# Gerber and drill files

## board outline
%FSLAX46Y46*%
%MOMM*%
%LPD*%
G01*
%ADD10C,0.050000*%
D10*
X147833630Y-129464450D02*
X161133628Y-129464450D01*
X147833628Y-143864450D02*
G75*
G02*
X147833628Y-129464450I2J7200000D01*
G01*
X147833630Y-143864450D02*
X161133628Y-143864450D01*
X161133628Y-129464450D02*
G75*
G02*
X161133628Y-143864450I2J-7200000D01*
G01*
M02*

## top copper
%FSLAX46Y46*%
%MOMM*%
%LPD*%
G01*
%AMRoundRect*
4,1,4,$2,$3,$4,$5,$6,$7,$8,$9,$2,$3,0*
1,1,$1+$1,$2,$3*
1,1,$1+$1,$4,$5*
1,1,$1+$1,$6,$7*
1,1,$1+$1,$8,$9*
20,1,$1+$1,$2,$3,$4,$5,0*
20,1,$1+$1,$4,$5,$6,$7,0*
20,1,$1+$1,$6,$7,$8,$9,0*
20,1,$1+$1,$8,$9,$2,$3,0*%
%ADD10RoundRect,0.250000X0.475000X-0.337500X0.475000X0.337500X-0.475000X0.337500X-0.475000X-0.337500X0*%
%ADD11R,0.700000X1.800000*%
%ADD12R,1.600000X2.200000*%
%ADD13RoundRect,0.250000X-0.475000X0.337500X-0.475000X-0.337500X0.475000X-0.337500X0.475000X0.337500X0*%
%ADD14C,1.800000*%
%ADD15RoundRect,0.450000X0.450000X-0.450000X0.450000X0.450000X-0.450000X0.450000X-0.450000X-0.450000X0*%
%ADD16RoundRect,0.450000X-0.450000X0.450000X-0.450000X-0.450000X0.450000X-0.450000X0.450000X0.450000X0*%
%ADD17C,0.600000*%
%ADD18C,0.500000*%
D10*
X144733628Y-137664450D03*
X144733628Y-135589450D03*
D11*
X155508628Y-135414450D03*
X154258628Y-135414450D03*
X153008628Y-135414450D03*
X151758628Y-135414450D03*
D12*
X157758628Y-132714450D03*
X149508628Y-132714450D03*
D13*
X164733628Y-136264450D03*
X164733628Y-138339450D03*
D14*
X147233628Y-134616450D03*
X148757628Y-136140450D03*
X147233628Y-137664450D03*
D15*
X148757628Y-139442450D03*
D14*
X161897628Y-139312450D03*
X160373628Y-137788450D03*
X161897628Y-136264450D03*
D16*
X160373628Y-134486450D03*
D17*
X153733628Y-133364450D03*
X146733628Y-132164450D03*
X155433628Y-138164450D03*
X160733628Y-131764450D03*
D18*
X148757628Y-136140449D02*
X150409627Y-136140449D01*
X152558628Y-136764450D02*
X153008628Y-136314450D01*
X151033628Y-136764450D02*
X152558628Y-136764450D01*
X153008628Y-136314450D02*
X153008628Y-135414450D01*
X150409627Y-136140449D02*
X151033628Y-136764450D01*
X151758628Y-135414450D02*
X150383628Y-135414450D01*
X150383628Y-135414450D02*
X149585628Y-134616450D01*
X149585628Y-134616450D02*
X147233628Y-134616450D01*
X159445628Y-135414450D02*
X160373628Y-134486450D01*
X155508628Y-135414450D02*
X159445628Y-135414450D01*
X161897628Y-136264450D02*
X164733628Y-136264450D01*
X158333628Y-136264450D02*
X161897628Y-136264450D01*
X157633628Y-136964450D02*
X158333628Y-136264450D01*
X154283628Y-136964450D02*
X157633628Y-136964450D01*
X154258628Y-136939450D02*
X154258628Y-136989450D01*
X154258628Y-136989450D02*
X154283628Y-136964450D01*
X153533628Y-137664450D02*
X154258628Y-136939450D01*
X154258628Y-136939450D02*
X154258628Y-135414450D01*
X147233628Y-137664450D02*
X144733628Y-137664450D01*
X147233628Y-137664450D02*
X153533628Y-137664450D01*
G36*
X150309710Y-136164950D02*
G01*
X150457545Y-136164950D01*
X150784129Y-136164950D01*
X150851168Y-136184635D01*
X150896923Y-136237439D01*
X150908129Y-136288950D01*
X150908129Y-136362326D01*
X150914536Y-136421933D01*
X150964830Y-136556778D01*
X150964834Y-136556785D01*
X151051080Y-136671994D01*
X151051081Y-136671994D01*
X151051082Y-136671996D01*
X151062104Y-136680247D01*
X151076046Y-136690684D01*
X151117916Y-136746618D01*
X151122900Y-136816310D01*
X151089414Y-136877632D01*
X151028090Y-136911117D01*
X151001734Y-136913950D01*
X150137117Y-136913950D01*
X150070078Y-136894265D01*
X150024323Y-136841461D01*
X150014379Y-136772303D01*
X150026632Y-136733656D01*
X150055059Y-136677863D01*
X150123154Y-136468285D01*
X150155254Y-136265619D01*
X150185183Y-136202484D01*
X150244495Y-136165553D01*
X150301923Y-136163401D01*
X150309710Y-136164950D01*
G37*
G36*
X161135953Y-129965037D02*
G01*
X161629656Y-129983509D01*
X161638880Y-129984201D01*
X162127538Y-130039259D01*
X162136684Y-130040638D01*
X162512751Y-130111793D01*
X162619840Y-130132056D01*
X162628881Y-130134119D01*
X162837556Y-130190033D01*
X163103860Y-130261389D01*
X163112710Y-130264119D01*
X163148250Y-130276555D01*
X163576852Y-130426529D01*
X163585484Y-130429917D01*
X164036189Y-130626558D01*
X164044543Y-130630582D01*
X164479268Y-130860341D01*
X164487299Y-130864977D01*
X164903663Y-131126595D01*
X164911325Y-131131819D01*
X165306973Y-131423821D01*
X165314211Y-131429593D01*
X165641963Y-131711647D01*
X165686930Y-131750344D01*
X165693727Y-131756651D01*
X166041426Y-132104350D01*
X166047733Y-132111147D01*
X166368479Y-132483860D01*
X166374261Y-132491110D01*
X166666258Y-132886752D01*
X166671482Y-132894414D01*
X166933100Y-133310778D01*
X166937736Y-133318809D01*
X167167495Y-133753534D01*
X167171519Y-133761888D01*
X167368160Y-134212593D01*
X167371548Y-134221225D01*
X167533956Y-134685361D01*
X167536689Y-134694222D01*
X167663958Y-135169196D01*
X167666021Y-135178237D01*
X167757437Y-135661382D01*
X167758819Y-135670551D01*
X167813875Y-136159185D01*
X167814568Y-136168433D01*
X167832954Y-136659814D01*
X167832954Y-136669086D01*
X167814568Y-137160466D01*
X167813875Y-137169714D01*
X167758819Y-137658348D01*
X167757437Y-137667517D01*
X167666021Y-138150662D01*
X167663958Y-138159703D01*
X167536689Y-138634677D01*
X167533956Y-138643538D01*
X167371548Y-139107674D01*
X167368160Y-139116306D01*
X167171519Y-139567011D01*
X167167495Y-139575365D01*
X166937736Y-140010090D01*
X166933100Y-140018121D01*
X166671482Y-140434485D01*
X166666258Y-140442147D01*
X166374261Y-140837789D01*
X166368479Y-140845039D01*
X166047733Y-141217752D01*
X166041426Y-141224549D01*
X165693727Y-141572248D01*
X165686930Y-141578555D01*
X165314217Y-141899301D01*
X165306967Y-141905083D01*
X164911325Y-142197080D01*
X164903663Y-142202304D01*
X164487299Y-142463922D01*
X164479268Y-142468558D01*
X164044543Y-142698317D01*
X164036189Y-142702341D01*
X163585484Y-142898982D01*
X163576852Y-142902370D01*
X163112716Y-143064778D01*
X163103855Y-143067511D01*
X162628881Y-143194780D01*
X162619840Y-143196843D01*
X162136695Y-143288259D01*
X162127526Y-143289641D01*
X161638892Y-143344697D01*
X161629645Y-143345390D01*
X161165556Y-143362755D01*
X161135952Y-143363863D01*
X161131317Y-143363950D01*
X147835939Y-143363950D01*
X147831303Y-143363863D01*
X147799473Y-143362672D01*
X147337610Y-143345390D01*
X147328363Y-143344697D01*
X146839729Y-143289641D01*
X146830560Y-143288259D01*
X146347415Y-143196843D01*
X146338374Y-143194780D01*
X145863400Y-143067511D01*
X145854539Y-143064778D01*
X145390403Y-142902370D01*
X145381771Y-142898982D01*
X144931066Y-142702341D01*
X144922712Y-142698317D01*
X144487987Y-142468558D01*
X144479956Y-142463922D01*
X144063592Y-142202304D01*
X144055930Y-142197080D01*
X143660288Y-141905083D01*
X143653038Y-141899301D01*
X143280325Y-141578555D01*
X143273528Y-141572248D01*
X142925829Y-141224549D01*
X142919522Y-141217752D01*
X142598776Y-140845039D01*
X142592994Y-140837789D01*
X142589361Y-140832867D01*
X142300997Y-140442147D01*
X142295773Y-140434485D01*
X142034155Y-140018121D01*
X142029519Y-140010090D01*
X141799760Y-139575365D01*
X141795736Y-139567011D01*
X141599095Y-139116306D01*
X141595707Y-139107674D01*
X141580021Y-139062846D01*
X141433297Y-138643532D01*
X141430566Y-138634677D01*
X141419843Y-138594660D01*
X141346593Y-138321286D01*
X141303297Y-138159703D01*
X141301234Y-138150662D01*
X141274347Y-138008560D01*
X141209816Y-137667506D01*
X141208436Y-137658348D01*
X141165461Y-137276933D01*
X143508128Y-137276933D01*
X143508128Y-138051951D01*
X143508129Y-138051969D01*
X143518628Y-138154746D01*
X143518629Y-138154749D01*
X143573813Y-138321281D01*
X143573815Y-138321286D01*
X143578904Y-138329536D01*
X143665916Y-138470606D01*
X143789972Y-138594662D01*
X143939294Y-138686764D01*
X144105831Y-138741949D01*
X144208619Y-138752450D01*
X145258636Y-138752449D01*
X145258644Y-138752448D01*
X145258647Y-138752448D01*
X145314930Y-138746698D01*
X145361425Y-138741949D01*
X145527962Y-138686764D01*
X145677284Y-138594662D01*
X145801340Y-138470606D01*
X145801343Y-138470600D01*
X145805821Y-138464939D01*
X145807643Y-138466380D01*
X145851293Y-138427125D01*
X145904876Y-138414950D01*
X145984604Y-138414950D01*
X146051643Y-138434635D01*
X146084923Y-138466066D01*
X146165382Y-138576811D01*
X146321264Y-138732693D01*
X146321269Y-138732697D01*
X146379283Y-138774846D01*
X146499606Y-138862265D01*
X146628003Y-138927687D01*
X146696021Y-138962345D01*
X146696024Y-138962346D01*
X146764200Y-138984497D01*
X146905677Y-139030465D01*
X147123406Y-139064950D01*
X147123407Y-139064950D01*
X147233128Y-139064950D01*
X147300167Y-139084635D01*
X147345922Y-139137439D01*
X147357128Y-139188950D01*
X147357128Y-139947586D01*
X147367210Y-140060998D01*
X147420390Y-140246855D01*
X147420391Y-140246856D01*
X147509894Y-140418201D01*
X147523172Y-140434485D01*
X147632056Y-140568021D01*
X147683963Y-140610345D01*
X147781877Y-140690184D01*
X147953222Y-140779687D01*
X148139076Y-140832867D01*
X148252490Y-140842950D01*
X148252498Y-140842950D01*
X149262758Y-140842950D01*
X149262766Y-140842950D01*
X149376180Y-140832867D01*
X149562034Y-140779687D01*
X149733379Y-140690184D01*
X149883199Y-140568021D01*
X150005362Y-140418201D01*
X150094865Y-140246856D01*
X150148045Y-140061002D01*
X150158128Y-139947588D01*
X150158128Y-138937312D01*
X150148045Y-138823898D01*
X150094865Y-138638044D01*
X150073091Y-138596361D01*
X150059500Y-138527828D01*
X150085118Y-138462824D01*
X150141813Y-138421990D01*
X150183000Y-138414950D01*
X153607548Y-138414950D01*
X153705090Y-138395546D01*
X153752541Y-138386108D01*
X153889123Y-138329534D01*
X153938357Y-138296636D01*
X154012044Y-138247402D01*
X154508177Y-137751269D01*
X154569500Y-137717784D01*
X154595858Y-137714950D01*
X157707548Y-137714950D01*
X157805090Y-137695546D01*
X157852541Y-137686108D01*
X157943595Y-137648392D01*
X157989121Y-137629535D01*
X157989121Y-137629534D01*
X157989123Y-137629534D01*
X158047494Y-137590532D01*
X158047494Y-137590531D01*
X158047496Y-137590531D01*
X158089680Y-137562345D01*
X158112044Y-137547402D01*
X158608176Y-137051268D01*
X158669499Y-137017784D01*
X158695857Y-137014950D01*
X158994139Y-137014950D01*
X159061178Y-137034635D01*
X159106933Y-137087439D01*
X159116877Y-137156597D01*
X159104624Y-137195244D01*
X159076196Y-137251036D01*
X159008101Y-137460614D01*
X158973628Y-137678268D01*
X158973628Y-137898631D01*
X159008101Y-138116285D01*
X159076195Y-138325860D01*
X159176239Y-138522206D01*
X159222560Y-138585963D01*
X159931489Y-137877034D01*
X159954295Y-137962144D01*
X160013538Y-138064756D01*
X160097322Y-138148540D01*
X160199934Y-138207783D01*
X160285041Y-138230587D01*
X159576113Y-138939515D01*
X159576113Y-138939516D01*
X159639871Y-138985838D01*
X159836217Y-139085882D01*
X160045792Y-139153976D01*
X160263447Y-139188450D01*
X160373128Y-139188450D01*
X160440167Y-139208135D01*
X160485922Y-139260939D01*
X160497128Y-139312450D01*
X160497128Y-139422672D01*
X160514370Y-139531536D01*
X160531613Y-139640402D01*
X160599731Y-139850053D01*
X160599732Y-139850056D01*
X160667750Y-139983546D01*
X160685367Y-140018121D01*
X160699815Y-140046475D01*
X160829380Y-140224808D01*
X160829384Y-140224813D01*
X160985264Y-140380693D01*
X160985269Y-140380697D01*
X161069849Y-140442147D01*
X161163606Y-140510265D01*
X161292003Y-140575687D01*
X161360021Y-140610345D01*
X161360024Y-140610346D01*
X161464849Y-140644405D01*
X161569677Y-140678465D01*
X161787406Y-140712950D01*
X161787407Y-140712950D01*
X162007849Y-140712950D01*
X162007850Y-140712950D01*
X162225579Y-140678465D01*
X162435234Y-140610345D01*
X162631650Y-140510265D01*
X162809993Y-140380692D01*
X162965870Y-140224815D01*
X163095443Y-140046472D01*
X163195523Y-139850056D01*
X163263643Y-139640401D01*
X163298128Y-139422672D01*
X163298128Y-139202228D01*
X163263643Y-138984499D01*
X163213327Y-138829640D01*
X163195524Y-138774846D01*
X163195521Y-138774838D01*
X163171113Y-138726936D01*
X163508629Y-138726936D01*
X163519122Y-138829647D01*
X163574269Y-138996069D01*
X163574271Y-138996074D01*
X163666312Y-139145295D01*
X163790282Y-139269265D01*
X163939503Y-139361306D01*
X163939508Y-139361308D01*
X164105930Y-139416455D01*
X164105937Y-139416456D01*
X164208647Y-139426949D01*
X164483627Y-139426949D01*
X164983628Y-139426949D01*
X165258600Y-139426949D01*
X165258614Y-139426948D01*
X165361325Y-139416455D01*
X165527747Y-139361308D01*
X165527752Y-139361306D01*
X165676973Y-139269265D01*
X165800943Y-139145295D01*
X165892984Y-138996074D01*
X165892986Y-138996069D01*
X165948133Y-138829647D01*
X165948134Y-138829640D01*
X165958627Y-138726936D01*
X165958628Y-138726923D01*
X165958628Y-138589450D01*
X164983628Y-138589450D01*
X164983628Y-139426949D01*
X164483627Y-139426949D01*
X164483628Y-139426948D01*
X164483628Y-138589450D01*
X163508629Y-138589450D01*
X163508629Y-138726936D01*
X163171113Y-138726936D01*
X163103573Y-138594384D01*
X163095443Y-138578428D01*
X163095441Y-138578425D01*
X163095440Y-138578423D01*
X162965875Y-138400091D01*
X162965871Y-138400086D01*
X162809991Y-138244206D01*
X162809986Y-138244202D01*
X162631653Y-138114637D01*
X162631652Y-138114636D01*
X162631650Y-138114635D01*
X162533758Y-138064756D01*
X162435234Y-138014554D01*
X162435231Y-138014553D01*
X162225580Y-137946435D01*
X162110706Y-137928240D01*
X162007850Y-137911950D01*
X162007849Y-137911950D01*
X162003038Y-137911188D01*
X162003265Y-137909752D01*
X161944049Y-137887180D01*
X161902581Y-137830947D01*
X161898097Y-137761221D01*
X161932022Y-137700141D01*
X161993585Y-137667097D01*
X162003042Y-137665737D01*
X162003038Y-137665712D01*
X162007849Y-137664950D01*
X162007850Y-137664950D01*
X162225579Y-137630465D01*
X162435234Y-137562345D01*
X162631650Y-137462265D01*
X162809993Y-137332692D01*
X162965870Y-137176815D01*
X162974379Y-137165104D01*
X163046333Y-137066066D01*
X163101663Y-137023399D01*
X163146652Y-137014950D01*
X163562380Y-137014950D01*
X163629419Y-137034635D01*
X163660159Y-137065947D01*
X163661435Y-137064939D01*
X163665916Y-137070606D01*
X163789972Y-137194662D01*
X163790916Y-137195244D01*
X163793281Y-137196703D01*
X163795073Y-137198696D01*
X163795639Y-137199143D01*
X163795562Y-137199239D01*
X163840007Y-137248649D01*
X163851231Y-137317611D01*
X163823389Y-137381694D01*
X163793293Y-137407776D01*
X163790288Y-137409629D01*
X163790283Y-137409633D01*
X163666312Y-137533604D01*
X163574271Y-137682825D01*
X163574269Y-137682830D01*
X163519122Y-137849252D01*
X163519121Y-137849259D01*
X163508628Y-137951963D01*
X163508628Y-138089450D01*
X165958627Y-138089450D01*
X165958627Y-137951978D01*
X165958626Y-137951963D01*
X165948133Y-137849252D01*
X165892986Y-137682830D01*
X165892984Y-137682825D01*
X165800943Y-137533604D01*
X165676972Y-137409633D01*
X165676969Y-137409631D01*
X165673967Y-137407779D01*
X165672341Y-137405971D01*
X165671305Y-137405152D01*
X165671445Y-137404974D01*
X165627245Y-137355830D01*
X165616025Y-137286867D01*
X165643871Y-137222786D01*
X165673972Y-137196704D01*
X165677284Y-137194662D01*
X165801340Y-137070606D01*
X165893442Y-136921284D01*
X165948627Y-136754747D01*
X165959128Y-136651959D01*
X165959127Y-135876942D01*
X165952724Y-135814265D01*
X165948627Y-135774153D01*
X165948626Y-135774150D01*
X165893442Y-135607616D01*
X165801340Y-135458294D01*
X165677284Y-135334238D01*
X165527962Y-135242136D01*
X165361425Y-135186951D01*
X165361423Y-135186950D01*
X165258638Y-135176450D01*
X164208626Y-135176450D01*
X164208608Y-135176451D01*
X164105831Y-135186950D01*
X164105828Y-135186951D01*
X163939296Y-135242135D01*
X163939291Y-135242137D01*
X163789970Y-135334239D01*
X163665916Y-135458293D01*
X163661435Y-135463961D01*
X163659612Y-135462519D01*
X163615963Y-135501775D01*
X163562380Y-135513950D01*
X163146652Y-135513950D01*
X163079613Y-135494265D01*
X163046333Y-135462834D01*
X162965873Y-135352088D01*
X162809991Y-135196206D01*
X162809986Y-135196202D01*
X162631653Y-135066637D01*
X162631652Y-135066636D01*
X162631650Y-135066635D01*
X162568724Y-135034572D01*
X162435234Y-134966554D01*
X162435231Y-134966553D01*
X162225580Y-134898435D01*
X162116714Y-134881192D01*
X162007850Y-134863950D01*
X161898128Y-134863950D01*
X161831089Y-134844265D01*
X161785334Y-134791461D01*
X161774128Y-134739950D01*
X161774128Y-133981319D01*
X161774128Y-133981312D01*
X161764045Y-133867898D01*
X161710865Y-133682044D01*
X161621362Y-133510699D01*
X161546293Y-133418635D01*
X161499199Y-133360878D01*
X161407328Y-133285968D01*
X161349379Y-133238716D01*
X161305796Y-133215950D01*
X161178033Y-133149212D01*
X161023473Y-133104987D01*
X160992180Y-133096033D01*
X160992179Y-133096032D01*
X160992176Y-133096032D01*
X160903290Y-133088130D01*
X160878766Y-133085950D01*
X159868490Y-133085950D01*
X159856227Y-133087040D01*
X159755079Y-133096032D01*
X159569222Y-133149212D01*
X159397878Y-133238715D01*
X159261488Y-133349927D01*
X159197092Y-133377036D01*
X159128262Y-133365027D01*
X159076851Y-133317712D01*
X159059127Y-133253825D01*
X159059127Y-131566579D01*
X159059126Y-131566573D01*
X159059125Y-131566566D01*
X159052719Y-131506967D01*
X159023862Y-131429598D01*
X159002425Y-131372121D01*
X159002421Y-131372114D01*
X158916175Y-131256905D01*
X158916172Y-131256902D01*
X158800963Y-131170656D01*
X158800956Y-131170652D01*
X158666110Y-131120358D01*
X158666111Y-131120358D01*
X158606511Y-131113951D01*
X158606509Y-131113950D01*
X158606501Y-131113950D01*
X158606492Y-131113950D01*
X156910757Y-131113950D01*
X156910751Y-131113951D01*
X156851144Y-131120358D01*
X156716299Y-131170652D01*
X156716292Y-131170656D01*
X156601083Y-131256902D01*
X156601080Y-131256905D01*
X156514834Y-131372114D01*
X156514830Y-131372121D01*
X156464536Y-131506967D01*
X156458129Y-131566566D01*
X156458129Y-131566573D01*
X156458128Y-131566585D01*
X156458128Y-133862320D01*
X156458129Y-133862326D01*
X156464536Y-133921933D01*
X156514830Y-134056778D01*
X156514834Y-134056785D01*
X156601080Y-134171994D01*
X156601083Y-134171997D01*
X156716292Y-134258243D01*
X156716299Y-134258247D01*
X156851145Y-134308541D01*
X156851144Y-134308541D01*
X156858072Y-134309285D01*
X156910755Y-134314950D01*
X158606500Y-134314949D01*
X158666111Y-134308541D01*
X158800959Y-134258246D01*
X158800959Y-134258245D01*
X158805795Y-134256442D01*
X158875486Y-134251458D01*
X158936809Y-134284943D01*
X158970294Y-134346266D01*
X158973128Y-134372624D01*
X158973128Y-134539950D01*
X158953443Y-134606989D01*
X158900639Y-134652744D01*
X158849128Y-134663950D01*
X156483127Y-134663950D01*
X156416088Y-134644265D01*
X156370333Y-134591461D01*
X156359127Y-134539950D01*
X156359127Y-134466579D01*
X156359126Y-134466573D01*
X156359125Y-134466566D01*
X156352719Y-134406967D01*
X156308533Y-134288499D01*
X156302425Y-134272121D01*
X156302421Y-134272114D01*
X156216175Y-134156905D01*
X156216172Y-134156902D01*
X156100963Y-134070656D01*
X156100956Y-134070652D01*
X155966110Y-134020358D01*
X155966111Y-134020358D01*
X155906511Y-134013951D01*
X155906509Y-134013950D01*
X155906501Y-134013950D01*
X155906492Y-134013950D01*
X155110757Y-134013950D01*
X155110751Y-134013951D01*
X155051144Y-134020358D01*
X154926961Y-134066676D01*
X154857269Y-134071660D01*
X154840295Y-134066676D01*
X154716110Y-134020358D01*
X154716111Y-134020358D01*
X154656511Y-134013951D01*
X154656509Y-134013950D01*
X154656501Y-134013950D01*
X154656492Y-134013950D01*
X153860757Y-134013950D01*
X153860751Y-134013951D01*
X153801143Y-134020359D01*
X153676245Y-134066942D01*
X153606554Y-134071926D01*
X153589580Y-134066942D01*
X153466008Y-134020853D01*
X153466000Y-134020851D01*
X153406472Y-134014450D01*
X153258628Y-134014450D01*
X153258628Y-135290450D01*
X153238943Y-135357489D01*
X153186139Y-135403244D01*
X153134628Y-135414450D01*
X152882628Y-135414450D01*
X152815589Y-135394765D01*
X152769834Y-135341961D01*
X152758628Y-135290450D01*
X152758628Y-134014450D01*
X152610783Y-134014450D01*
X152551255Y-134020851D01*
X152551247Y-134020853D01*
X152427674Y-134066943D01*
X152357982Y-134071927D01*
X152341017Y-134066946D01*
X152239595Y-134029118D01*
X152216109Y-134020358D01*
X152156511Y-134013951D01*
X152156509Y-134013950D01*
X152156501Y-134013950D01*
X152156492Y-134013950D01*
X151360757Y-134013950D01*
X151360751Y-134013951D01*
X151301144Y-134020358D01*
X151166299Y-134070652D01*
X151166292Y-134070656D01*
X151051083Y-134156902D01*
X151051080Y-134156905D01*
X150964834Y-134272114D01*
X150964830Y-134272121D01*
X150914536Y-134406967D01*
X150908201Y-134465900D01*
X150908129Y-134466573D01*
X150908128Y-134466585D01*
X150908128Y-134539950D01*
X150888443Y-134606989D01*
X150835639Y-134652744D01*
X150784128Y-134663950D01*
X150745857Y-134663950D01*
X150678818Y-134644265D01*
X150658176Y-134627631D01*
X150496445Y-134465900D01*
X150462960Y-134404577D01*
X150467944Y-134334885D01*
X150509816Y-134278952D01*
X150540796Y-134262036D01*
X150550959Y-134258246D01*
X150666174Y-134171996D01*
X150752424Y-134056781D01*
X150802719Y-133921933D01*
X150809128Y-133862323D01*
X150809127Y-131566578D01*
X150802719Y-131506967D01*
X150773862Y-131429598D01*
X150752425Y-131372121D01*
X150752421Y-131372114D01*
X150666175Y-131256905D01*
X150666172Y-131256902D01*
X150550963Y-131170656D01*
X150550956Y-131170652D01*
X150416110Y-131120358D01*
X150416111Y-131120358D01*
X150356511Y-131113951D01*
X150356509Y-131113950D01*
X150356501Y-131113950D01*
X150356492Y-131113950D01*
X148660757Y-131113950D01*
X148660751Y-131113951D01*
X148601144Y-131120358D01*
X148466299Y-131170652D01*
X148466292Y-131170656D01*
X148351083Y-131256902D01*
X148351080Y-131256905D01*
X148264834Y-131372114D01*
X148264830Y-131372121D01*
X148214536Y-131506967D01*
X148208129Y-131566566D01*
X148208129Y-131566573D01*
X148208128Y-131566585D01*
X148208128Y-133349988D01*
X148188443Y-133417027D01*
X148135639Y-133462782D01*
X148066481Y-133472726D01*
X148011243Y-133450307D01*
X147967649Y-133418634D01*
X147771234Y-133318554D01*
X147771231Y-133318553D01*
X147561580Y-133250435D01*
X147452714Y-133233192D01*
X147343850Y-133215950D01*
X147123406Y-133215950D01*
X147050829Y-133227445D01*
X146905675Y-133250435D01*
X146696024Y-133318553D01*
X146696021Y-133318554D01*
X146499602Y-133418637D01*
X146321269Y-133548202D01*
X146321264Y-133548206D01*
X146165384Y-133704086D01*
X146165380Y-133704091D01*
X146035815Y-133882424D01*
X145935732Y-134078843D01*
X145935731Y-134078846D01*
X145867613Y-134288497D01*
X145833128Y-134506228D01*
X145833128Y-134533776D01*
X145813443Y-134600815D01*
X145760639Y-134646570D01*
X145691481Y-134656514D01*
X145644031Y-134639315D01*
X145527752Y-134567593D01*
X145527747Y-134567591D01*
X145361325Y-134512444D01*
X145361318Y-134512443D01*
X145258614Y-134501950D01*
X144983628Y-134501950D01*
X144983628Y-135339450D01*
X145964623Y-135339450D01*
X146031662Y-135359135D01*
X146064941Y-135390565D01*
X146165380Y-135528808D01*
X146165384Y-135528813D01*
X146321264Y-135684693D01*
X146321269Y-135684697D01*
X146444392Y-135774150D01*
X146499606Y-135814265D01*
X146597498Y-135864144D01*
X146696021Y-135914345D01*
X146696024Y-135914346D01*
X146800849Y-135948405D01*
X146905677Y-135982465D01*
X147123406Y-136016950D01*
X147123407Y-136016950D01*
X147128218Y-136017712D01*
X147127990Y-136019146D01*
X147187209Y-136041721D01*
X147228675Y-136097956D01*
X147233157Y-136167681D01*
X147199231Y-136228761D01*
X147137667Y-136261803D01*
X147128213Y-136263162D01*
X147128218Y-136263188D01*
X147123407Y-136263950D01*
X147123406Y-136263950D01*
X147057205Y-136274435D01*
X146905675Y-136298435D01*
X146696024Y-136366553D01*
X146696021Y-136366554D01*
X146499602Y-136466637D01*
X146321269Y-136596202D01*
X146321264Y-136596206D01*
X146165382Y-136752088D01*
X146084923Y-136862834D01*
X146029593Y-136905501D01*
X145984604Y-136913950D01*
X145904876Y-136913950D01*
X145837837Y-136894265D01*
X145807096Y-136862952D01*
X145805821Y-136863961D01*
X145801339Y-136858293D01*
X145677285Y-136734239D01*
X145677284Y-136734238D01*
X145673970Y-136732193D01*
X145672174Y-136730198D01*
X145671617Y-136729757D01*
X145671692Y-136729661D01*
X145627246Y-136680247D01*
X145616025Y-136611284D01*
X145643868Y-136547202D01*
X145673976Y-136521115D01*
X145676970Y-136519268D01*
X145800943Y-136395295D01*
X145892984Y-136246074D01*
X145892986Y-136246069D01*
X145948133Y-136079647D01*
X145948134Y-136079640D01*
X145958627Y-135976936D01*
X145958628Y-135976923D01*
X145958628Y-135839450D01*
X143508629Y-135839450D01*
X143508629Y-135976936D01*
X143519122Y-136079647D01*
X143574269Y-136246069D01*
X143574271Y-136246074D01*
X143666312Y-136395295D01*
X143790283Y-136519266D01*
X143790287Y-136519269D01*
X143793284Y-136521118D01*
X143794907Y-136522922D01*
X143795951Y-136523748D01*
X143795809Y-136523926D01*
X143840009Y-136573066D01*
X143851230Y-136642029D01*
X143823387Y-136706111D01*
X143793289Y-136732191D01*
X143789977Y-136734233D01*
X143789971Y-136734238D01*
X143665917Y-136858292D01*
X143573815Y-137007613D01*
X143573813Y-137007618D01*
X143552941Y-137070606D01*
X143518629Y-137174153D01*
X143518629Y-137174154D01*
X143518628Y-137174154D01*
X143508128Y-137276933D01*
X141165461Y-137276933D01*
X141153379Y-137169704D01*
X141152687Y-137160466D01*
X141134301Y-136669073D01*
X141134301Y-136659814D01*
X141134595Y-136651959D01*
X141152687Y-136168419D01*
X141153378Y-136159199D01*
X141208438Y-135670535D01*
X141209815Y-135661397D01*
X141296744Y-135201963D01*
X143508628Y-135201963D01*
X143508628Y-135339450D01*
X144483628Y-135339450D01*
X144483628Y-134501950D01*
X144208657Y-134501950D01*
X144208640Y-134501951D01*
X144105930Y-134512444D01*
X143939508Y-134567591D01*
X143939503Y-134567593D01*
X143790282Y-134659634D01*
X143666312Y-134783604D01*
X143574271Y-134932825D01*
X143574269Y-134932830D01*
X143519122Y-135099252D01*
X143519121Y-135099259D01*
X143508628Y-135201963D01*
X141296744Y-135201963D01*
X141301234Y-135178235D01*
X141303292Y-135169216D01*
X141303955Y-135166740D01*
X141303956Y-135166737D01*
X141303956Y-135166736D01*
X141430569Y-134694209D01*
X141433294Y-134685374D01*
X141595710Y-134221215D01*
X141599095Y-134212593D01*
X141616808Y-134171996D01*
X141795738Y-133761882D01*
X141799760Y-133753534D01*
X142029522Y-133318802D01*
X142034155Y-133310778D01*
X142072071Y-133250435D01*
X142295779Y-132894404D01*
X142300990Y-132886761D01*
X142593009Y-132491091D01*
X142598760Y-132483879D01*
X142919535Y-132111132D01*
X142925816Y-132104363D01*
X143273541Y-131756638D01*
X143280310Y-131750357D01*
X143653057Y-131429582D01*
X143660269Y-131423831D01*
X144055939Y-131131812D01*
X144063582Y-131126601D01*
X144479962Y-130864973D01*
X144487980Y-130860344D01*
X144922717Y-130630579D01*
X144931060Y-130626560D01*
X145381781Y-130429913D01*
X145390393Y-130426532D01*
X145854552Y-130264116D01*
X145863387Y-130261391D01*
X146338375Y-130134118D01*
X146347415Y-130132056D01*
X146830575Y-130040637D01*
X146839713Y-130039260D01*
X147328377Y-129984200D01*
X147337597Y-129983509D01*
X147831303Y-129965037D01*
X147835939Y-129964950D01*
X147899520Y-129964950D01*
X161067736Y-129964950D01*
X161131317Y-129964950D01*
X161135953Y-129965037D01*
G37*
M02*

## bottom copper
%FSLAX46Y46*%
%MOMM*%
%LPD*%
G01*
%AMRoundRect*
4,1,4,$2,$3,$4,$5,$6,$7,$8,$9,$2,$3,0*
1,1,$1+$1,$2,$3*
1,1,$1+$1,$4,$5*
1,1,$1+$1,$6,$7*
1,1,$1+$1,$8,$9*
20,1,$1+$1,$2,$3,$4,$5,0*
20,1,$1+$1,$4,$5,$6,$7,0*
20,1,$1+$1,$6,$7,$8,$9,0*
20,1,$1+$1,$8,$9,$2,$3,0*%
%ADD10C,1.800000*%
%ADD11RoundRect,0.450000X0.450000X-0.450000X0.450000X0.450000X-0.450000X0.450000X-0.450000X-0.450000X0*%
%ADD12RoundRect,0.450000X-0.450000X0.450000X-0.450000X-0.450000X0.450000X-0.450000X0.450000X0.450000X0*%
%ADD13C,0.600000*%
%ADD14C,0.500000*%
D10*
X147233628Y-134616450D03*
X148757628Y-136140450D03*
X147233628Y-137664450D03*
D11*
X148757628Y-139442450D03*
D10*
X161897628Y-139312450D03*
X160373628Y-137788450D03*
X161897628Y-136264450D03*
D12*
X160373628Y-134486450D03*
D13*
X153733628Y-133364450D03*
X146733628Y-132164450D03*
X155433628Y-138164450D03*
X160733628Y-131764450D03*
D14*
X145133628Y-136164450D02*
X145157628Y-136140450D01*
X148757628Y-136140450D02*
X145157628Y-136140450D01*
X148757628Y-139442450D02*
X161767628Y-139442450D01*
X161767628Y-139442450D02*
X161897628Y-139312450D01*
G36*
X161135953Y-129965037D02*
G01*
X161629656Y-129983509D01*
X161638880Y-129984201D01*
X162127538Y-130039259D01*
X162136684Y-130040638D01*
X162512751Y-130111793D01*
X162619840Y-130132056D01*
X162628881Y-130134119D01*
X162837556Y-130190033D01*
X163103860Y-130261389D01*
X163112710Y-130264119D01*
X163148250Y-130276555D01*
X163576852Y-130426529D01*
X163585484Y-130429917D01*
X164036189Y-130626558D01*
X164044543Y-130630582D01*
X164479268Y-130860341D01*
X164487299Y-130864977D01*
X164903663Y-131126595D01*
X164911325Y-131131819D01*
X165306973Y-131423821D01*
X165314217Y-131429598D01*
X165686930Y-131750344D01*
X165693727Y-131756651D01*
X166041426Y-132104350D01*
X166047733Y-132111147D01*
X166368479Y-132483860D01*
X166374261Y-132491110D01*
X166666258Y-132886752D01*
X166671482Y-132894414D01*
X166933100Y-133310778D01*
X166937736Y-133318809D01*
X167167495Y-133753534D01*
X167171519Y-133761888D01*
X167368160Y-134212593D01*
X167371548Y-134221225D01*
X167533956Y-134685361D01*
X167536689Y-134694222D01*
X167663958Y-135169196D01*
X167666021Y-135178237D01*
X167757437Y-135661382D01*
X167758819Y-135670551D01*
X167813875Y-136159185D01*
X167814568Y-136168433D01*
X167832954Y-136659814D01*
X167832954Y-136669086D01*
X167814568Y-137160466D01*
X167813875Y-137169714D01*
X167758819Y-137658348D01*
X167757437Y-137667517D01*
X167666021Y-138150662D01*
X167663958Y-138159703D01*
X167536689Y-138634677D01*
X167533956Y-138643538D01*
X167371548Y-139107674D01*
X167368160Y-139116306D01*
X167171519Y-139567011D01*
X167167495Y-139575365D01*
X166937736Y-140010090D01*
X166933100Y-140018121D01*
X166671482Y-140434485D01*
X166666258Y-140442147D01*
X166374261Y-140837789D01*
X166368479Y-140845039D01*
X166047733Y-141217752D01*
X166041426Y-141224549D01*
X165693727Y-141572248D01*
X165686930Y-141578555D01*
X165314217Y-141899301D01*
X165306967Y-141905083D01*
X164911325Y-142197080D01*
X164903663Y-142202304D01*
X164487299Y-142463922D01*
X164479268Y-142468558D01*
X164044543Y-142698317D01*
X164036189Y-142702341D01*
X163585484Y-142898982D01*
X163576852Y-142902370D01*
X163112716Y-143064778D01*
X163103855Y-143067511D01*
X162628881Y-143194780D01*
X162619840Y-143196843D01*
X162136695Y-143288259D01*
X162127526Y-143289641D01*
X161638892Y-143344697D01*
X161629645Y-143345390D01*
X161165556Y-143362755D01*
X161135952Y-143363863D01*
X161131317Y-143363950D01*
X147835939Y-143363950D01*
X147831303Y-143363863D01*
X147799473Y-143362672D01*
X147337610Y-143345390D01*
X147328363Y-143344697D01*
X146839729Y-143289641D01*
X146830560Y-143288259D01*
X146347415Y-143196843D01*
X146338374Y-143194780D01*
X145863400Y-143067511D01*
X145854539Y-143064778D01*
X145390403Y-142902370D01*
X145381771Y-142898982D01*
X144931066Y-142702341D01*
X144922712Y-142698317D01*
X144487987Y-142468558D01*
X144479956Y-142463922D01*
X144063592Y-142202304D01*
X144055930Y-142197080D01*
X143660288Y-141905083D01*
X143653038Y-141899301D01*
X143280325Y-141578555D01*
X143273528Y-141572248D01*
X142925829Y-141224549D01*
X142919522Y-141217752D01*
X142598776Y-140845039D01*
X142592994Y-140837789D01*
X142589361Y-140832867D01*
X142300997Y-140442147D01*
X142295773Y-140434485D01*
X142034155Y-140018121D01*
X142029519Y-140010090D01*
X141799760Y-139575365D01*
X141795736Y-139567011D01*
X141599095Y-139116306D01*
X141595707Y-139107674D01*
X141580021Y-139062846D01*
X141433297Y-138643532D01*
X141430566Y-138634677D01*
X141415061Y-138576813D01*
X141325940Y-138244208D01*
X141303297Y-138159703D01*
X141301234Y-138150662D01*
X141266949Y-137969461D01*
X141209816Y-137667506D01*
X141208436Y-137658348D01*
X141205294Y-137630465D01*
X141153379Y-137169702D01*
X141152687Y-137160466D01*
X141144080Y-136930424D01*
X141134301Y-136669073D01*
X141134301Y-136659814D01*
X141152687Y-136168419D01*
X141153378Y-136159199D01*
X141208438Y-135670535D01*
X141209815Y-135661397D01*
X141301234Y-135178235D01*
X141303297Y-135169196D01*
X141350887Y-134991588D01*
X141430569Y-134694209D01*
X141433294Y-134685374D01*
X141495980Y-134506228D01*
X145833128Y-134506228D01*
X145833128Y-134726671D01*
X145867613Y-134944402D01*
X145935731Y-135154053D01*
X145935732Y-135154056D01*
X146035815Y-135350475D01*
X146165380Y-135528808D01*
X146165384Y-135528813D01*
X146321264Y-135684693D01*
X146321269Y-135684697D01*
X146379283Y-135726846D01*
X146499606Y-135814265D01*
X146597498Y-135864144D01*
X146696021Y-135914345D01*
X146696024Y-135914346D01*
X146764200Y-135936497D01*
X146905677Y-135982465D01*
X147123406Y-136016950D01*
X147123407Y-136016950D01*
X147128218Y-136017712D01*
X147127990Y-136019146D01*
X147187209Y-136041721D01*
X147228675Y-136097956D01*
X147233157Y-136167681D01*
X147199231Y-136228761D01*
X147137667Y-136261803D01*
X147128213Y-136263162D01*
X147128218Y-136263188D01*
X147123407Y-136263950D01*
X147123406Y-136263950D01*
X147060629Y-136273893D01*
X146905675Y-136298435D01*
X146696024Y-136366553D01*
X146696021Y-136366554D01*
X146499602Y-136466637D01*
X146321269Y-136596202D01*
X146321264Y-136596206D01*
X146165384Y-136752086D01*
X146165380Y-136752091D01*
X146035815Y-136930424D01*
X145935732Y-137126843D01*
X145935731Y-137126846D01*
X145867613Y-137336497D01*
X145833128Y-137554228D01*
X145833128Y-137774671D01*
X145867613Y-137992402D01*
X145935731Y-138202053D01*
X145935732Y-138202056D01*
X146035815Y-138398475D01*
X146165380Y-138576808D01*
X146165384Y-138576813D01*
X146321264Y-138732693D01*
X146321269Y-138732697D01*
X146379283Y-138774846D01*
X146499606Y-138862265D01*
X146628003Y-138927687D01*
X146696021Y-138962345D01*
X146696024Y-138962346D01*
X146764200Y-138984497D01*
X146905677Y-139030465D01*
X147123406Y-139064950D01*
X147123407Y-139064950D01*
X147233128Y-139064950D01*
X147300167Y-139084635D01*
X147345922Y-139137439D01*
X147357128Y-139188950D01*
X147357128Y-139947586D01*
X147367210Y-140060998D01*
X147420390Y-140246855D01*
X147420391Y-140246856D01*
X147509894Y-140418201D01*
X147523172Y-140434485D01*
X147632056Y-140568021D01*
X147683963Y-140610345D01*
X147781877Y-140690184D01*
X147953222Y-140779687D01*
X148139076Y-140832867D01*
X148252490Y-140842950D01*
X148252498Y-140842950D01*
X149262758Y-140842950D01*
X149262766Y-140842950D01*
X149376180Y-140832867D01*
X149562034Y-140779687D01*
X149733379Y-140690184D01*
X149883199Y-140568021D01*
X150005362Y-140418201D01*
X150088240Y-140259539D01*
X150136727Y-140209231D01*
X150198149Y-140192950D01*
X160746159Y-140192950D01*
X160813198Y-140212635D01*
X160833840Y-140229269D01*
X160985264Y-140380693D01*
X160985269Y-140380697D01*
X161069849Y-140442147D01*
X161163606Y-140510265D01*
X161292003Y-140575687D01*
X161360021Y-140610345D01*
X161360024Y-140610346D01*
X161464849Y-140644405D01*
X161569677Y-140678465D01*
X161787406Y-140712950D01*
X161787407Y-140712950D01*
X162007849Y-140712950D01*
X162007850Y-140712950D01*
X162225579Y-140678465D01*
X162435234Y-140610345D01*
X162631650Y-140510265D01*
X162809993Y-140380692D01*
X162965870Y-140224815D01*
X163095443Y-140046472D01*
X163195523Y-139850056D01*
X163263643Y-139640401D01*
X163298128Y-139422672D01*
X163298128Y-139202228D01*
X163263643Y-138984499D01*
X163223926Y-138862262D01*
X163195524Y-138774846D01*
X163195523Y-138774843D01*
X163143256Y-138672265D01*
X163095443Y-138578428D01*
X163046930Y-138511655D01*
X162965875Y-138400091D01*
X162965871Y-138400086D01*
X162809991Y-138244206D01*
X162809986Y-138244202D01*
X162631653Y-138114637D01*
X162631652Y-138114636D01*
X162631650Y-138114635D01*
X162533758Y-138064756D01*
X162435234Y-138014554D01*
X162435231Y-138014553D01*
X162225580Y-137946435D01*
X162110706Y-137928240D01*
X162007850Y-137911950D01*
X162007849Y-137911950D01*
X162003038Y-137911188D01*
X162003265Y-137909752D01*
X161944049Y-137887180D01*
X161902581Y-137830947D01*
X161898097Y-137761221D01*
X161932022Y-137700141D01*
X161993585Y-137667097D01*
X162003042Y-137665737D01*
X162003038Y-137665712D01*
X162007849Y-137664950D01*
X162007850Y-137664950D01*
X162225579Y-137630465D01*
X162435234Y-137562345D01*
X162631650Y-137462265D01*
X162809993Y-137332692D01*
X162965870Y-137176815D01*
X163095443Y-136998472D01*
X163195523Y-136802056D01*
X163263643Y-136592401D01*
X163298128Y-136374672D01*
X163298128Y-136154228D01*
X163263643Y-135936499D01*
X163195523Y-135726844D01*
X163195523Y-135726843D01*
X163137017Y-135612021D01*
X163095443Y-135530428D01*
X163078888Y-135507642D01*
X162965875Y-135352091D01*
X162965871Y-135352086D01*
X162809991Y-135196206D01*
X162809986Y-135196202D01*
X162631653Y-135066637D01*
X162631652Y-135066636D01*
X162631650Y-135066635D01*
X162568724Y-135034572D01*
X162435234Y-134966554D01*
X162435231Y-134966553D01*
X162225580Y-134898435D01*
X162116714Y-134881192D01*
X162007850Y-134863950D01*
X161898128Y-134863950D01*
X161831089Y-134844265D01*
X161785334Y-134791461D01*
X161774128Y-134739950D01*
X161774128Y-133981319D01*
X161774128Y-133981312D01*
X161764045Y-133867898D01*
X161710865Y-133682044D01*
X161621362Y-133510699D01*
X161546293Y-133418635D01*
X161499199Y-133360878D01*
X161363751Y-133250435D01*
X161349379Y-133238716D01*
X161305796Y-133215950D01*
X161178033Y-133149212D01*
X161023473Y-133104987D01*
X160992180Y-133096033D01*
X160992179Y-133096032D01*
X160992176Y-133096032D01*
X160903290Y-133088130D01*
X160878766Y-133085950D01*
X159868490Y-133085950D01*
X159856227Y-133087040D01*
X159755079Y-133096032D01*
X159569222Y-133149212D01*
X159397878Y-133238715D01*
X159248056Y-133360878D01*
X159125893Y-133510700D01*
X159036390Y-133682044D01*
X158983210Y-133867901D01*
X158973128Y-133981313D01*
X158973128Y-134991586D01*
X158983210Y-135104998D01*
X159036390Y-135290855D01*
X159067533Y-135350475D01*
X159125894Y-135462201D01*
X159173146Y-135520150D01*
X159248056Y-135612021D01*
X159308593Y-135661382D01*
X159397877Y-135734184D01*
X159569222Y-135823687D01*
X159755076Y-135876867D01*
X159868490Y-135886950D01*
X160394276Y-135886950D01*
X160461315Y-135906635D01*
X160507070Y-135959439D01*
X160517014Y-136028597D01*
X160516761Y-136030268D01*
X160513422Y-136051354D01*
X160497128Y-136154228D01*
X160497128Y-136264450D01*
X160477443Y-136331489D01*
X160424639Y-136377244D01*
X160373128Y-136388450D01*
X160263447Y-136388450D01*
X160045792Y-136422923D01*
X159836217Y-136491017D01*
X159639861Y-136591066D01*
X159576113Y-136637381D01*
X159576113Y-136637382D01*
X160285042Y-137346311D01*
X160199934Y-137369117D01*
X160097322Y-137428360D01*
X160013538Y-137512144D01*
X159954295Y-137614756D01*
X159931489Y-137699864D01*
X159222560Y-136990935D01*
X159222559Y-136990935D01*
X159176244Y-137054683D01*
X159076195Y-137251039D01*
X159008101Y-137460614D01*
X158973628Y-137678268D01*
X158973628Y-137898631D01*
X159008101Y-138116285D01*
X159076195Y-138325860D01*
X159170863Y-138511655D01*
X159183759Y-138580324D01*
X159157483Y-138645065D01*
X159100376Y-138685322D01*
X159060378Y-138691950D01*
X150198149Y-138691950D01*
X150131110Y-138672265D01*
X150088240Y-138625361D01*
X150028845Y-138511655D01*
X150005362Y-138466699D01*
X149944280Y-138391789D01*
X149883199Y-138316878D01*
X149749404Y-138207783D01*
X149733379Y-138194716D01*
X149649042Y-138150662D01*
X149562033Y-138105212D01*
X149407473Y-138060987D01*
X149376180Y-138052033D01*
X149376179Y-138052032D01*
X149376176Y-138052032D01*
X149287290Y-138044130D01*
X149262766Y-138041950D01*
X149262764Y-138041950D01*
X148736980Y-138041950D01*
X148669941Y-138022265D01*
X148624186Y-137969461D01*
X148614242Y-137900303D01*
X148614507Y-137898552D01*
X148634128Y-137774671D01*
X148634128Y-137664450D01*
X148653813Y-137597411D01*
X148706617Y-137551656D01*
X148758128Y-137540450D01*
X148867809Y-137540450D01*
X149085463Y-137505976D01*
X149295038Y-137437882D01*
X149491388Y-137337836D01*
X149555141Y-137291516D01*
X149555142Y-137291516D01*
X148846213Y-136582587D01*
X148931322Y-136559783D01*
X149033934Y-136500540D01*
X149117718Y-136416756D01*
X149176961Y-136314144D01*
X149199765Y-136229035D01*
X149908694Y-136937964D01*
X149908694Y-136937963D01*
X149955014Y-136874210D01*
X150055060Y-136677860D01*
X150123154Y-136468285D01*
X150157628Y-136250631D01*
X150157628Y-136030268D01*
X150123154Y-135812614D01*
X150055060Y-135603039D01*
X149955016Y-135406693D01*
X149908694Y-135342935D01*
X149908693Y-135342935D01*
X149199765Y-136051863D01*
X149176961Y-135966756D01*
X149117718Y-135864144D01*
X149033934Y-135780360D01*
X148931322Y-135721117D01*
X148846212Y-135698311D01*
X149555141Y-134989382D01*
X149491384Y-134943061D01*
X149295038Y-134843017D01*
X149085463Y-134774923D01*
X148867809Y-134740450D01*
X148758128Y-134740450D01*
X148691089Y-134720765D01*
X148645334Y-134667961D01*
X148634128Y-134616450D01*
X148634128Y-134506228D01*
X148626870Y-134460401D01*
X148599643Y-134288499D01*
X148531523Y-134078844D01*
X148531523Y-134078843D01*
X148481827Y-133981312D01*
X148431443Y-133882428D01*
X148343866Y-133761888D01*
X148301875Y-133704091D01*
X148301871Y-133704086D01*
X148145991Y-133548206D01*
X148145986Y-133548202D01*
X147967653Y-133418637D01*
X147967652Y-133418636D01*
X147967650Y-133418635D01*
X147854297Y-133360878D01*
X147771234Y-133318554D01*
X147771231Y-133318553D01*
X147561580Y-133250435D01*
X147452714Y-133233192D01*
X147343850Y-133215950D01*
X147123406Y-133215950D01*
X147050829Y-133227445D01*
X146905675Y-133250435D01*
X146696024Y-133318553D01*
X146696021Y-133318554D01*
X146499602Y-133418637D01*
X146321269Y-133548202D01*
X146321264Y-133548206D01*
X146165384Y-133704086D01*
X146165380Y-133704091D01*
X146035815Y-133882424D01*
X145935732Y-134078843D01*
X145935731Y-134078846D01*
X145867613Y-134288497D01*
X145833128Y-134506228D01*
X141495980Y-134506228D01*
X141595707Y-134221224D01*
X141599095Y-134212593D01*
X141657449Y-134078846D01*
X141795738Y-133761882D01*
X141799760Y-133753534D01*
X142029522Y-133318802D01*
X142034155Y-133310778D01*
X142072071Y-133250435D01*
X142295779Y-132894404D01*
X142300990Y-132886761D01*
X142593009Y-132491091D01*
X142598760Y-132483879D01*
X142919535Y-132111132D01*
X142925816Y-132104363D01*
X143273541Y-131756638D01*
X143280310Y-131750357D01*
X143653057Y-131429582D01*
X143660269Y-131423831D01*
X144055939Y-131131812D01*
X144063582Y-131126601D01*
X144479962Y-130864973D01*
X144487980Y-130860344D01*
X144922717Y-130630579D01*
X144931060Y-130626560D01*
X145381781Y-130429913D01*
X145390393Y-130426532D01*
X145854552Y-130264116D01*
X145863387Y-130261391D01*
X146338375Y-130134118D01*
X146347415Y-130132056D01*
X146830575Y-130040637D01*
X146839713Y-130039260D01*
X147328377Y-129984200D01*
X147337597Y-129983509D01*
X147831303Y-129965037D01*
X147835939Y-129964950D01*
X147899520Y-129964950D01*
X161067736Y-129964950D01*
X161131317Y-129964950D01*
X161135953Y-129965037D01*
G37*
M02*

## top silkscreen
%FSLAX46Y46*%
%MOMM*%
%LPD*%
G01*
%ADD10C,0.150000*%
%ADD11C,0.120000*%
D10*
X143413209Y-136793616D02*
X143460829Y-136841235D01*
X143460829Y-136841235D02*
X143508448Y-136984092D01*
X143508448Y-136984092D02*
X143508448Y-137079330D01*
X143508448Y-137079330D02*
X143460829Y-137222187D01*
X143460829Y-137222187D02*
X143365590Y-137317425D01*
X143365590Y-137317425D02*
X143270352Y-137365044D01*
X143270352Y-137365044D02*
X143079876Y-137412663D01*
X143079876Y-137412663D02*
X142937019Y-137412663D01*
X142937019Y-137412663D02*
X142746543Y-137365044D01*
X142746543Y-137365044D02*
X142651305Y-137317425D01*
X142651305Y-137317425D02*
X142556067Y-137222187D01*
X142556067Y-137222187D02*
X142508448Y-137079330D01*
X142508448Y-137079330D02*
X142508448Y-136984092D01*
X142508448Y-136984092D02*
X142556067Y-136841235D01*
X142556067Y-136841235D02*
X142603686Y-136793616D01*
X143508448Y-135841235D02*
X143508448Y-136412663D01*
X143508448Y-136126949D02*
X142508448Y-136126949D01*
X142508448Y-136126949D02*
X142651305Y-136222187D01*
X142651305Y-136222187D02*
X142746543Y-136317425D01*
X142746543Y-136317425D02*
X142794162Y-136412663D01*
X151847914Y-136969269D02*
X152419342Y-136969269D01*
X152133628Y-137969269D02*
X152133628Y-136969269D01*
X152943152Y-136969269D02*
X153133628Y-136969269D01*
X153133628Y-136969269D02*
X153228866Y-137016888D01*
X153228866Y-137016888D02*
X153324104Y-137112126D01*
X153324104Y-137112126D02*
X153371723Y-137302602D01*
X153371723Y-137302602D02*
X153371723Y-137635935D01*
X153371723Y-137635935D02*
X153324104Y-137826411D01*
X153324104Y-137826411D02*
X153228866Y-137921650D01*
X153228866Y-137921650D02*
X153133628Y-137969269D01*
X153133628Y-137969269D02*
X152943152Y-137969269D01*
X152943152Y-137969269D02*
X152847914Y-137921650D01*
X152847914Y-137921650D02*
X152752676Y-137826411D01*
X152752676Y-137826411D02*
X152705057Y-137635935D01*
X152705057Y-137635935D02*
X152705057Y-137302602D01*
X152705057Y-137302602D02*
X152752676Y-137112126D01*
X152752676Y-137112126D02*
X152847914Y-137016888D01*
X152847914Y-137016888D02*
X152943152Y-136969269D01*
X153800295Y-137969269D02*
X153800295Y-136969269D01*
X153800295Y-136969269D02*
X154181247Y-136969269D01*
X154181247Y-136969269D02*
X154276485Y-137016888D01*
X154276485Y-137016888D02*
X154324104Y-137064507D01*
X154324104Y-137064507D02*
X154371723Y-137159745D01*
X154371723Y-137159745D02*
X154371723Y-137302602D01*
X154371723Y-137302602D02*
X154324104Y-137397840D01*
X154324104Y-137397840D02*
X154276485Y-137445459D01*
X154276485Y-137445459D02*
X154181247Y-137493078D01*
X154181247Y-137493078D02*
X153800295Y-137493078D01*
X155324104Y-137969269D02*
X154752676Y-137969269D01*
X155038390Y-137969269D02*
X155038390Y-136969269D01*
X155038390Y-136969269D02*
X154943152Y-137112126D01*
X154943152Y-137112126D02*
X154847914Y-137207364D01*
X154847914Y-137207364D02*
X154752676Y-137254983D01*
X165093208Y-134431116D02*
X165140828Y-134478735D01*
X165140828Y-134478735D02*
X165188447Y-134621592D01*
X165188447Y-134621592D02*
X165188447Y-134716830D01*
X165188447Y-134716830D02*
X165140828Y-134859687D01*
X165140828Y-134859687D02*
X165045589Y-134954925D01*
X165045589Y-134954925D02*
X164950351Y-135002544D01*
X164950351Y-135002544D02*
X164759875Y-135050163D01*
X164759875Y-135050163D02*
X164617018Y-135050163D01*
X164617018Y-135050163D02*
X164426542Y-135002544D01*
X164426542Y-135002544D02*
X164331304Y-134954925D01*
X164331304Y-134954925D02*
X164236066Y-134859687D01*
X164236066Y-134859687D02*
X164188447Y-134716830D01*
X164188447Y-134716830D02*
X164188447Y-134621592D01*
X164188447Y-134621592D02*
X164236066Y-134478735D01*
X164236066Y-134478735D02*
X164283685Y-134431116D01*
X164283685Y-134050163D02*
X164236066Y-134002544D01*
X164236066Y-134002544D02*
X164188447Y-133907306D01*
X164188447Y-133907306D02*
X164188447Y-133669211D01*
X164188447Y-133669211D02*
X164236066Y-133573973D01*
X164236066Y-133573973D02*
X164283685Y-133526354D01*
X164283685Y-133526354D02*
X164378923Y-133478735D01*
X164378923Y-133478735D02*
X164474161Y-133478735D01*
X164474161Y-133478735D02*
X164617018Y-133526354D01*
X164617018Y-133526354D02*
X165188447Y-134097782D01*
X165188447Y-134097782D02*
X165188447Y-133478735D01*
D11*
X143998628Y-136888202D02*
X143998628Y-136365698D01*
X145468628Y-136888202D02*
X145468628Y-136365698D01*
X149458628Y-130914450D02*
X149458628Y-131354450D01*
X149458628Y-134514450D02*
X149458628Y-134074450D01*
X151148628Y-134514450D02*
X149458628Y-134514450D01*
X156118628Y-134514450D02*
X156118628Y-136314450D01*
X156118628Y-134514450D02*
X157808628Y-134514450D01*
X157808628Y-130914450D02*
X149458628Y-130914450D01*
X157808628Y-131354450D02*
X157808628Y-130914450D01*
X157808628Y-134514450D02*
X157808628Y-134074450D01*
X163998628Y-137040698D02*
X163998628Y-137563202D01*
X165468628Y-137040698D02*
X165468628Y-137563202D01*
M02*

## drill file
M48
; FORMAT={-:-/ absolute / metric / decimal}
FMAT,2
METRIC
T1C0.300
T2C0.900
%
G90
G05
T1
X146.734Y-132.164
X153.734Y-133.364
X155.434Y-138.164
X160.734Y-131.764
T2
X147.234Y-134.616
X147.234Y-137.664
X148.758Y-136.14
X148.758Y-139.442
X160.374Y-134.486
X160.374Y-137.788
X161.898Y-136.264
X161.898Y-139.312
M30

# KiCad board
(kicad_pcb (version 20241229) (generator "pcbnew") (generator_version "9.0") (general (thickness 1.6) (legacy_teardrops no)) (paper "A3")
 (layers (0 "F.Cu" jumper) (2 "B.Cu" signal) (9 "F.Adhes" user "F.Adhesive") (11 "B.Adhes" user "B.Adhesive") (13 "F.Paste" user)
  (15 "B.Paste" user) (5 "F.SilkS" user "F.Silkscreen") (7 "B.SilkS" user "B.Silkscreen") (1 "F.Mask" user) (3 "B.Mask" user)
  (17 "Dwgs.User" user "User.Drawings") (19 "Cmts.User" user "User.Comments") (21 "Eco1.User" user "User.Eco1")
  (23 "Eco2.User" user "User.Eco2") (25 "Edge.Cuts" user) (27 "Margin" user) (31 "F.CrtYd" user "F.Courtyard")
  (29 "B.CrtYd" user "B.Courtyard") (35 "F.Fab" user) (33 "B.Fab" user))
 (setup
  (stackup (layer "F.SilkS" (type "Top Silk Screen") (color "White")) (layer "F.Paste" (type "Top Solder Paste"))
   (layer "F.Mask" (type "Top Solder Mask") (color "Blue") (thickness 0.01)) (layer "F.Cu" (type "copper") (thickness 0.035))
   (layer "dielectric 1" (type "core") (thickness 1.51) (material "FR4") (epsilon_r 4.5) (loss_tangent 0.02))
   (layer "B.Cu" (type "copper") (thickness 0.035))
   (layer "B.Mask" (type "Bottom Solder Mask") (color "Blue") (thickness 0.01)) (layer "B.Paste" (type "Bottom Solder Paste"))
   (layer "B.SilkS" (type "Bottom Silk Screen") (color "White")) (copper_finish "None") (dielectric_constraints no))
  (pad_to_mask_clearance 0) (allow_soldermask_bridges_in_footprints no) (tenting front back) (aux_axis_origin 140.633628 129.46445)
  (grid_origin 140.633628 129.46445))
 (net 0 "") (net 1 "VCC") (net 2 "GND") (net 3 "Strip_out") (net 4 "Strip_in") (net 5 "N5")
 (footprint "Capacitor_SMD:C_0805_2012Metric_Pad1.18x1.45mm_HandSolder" (layer "F.Cu") (at 144.733628 136.62695 90)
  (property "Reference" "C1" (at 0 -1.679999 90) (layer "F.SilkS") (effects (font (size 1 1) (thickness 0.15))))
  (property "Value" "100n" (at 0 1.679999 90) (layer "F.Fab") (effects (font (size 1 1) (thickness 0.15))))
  (fp_line (start -0.261252 -0.735) (end 0.261252 -0.735) (stroke (width 0.12) (type solid)) (layer "F.SilkS"))
  (fp_line (start -0.261252 0.735) (end 0.261252 0.735) (stroke (width 0.12) (type solid)) (layer "F.SilkS"))
  (pad "1" smd roundrect (at -1.0375 0 90) (size 1.175 1.45) (layers "F.Cu" "F.Mask" "F.Paste") (roundrect_rratio 0.212766) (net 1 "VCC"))
  (pad "2" smd roundrect (at 1.0375 0 90) (size 1.175 1.45) (layers "F.Cu" "F.Mask" "F.Paste") (roundrect_rratio 0.212766) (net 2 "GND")))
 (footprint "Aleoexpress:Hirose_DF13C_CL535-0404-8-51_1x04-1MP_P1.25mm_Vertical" (layer "F.Cu") (at 153.633628 133.96445 180)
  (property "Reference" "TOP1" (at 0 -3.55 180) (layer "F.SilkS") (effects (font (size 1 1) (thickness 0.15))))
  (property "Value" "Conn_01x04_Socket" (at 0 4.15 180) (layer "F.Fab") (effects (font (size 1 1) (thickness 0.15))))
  (fp_line (start 4.175 3.05) (end 4.175 2.61) (stroke (width 0.12) (type solid)) (layer "F.SilkS"))
  (fp_line (start 4.175 -0.55) (end 4.175 -0.11) (stroke (width 0.12) (type solid)) (layer "F.SilkS"))
  (fp_line (start 2.485 -0.55) (end 4.175 -0.55) (stroke (width 0.12) (type solid)) (layer "F.SilkS"))
  (fp_line (start -2.485 -0.55) (end -2.485 -2.35) (stroke (width 0.12) (type solid)) (layer "F.SilkS"))
  (fp_line (start -2.485 -0.55) (end -4.175 -0.55) (stroke (width 0.12) (type solid)) (layer "F.SilkS"))
  (fp_line (start -4.175 3.05) (end 4.175 3.05) (stroke (width 0.12) (type solid)) (layer "F.SilkS"))
  (fp_line (start -4.175 2.61) (end -4.175 3.05) (stroke (width 0.12) (type solid)) (layer "F.SilkS"))
  (fp_line (start -4.175 -0.55) (end -4.175 -0.11) (stroke (width 0.12) (type solid)) (layer "F.SilkS"))
  (pad "1" smd rect (at -1.875 -1.45 180) (size 0.7 1.8) (layers "F.Cu" "F.Mask" "F.Paste") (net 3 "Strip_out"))
  (pad "2" smd rect (at -0.625 -1.45 180) (size 0.7 1.8) (layers "F.Cu" "F.Mask" "F.Paste") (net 1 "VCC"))
  (pad "3" smd rect (at 0.625 -1.45 180) (size 0.7 1.8) (layers "F.Cu" "F.Mask" "F.Paste") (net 2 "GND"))
  (pad "4" smd rect (at 1.875 -1.45 180) (size 0.7 1.8) (layers "F.Cu" "F.Mask" "F.Paste") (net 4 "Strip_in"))
  (pad "MP" smd rect (at -4.125 1.25 180) (size 1.6 2.2) (layers "F.Cu" "F.Mask" "F.Paste"))
  (pad "MP" smd rect (at 4.125 1.25 180) (size 1.6 2.2) (layers "F.Cu" "F.Mask" "F.Paste")))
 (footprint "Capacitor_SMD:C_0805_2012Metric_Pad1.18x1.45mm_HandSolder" (layer "F.Cu") (at 164.733628 137.30195 -90)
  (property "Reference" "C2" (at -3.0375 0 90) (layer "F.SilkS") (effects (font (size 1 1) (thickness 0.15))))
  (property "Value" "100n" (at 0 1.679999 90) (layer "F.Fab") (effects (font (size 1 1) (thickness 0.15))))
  (fp_line (start -0.261252 0.735) (end 0.261252 0.735) (stroke (width 0.12) (type solid)) (layer "F.SilkS"))
  (fp_line (start -0.261252 -0.735) (end 0.261252 -0.735) (stroke (width 0.12) (type solid)) (layer "F.SilkS"))
  (pad "1" smd roundrect (at -1.0375 0 270) (size 1.175 1.45) (layers "F.Cu" "F.Mask" "F.Paste") (roundrect_rratio 0.212766) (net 1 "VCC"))
  (pad "2" smd roundrect (at 1.0375 0 270) (size 1.175 1.45) (layers "F.Cu" "F.Mask" "F.Paste") (roundrect_rratio 0.212766) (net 2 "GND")))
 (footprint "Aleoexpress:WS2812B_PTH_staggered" (layer "B.Cu") (at 148.757628 139.44245 90)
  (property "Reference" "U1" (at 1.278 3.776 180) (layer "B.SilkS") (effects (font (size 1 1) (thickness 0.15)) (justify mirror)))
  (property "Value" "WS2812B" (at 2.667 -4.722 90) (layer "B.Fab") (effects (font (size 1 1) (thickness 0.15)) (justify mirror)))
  (pad "1" thru_hole circle (at 4.826 -1.524 90) (size 1.8 1.8) (drill 0.9) (layers "*.Cu" "*.Mask") (remove_unused_layers no)
   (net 4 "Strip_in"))
  (pad "2" thru_hole circle (at 3.302 0 90) (size 1.8 1.8) (drill 0.9) (layers "*.Cu" "*.Mask") (remove_unused_layers no) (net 2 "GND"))
  (pad "3" thru_hole circle (at 1.778 -1.524 90) (size 1.8 1.8) (drill 0.9) (layers "*.Cu" "*.Mask") (remove_unused_layers no) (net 1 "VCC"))
  (pad "4" thru_hole roundrect (at 0 0 90) (size 1.8 1.8) (drill 0.9) (layers "*.Cu" "*.Mask") (remove_unused_layers no)
   (roundrect_rratio 0.25) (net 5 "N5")))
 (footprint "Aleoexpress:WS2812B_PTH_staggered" (layer "B.Cu") (at 160.373628 134.48645 -90)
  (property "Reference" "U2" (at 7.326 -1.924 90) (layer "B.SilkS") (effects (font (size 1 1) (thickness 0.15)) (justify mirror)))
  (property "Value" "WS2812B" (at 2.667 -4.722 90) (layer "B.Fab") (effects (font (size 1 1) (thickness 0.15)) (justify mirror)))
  (pad "1" thru_hole circle (at 4.826 -1.524 270) (size 1.8 1.8) (drill 0.9) (layers "*.Cu" "*.Mask") (remove_unused_layers no) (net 5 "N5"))
  (pad "2" thru_hole circle (at 3.302 0 270) (size 1.8 1.8) (drill 0.9) (layers "*.Cu" "*.Mask") (remove_unused_layers no) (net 2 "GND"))
  (pad "3" thru_hole circle (at 1.778 -1.524 270) (size 1.8 1.8) (drill 0.9) (layers "*.Cu" "*.Mask") (remove_unused_layers no)
   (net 1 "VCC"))
  (pad "4" thru_hole roundrect (at 0 0 270) (size 1.8 1.8) (drill 0.9) (layers "*.Cu" "*.Mask") (remove_unused_layers no)
   (roundrect_rratio 0.25) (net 3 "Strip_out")))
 (gr_line (start 147.83363 129.46445) (end 161.133628 129.46445) (stroke (width 0.05) (type default)) (layer "Edge.Cuts"))
 (gr_arc (start 147.833628 143.86445) (mid 140.633628 136.66445) (end 147.833628 129.46445) (stroke (width 0.05) (type default))
  (layer "Edge.Cuts"))
 (gr_line (start 147.83363 143.86445) (end 161.133628 143.86445) (stroke (width 0.05) (type default)) (layer "Edge.Cuts"))
 (gr_arc (start 161.133628 129.46445) (mid 168.333628 136.66445) (end 161.133628 143.86445) (stroke (width 0.05) (type default))
  (layer "Edge.Cuts"))
 (segment (start 148.757628 136.140449) (end 150.409627 136.140449) (width 0.5) (layer "F.Cu") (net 2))
 (segment (start 152.558628 136.76445) (end 153.008628 136.31445) (width 0.5) (layer "F.Cu") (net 2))
 (segment (start 151.033628 136.76445) (end 152.558628 136.76445) (width 0.5) (layer "F.Cu") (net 2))
 (segment (start 153.008628 136.31445) (end 153.008628 135.41445) (width 0.5) (layer "F.Cu") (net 2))
 (segment (start 150.409627 136.140449) (end 151.033628 136.76445) (width 0.5) (layer "F.Cu") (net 2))
 (via (at 153.733628 133.36445) (size 0.6) (drill 0.3) (layers "F.Cu" "B.Cu") (free yes) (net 2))
 (via (at 146.733628 132.16445) (size 0.6) (drill 0.3) (layers "F.Cu" "B.Cu") (free yes) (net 2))
 (via (at 155.433628 138.16445) (size 0.6) (drill 0.3) (layers "F.Cu" "B.Cu") (free yes) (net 2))
 (via (at 160.733628 131.76445) (size 0.6) (drill 0.3) (layers "F.Cu" "B.Cu") (free yes) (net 2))
 (segment (start 145.133628 136.16445) (end 145.157628 136.14045) (width 0.5) (layer "B.Cu") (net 2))
 (segment (start 148.757628 136.14045) (end 145.157628 136.14045) (width 0.5) (layer "B.Cu") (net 2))
 (segment (start 151.758628 135.41445) (end 150.383628 135.41445) (width 0.5) (layer "F.Cu") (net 4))
 (segment (start 150.383628 135.41445) (end 149.585628 134.61645) (width 0.5) (layer "F.Cu") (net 4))
 (segment (start 149.585628 134.61645) (end 147.233628 134.61645) (width 0.5) (layer "F.Cu") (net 4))
 (segment (start 148.757628 139.44245) (end 161.767628 139.44245) (width 0.5) (layer "B.Cu") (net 5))
 (segment (start 161.767628 139.44245) (end 161.897628 139.31245) (width 0.5) (layer "B.Cu") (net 5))
 (segment (start 159.445628 135.41445) (end 160.373628 134.48645) (width 0.5) (layer "F.Cu") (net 3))
 (segment (start 155.508628 135.41445) (end 159.445628 135.41445) (width 0.5) (layer "F.Cu") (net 3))
 (segment (start 161.897628 136.26445) (end 164.733628 136.26445) (width 0.5) (layer "F.Cu") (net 1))
 (segment (start 158.333628 136.26445) (end 161.897628 136.26445) (width 0.5) (layer "F.Cu") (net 1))
 (segment (start 157.633628 136.96445) (end 158.333628 136.26445) (width 0.5) (layer "F.Cu") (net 1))
 (segment (start 154.283628 136.96445) (end 157.633628 136.96445) (width 0.5) (layer "F.Cu") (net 1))
 (segment (start 154.258628 136.93945) (end 154.258628 136.98945) (width 0.5) (layer "F.Cu") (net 1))
 (segment (start 154.258628 136.98945) (end 154.283628 136.96445) (width 0.5) (layer "F.Cu") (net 1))
 (segment (start 153.533628 137.66445) (end 154.258628 136.93945) (width 0.5) (layer "F.Cu") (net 1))
 (segment (start 154.258628 136.93945) (end 154.258628 135.41445) (width 0.5) (layer "F.Cu") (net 1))
 (segment (start 147.233628 137.66445) (end 144.733628 137.66445) (width 0.5) (layer "F.Cu") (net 1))
 (segment (start 147.233628 137.66445) (end 153.533628 137.66445) (width 0.5) (layer "F.Cu") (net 1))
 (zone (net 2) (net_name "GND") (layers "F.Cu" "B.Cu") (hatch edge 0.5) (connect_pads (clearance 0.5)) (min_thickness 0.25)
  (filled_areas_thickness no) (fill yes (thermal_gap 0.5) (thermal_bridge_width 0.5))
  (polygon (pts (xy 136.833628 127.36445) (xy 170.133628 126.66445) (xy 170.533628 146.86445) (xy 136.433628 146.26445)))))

